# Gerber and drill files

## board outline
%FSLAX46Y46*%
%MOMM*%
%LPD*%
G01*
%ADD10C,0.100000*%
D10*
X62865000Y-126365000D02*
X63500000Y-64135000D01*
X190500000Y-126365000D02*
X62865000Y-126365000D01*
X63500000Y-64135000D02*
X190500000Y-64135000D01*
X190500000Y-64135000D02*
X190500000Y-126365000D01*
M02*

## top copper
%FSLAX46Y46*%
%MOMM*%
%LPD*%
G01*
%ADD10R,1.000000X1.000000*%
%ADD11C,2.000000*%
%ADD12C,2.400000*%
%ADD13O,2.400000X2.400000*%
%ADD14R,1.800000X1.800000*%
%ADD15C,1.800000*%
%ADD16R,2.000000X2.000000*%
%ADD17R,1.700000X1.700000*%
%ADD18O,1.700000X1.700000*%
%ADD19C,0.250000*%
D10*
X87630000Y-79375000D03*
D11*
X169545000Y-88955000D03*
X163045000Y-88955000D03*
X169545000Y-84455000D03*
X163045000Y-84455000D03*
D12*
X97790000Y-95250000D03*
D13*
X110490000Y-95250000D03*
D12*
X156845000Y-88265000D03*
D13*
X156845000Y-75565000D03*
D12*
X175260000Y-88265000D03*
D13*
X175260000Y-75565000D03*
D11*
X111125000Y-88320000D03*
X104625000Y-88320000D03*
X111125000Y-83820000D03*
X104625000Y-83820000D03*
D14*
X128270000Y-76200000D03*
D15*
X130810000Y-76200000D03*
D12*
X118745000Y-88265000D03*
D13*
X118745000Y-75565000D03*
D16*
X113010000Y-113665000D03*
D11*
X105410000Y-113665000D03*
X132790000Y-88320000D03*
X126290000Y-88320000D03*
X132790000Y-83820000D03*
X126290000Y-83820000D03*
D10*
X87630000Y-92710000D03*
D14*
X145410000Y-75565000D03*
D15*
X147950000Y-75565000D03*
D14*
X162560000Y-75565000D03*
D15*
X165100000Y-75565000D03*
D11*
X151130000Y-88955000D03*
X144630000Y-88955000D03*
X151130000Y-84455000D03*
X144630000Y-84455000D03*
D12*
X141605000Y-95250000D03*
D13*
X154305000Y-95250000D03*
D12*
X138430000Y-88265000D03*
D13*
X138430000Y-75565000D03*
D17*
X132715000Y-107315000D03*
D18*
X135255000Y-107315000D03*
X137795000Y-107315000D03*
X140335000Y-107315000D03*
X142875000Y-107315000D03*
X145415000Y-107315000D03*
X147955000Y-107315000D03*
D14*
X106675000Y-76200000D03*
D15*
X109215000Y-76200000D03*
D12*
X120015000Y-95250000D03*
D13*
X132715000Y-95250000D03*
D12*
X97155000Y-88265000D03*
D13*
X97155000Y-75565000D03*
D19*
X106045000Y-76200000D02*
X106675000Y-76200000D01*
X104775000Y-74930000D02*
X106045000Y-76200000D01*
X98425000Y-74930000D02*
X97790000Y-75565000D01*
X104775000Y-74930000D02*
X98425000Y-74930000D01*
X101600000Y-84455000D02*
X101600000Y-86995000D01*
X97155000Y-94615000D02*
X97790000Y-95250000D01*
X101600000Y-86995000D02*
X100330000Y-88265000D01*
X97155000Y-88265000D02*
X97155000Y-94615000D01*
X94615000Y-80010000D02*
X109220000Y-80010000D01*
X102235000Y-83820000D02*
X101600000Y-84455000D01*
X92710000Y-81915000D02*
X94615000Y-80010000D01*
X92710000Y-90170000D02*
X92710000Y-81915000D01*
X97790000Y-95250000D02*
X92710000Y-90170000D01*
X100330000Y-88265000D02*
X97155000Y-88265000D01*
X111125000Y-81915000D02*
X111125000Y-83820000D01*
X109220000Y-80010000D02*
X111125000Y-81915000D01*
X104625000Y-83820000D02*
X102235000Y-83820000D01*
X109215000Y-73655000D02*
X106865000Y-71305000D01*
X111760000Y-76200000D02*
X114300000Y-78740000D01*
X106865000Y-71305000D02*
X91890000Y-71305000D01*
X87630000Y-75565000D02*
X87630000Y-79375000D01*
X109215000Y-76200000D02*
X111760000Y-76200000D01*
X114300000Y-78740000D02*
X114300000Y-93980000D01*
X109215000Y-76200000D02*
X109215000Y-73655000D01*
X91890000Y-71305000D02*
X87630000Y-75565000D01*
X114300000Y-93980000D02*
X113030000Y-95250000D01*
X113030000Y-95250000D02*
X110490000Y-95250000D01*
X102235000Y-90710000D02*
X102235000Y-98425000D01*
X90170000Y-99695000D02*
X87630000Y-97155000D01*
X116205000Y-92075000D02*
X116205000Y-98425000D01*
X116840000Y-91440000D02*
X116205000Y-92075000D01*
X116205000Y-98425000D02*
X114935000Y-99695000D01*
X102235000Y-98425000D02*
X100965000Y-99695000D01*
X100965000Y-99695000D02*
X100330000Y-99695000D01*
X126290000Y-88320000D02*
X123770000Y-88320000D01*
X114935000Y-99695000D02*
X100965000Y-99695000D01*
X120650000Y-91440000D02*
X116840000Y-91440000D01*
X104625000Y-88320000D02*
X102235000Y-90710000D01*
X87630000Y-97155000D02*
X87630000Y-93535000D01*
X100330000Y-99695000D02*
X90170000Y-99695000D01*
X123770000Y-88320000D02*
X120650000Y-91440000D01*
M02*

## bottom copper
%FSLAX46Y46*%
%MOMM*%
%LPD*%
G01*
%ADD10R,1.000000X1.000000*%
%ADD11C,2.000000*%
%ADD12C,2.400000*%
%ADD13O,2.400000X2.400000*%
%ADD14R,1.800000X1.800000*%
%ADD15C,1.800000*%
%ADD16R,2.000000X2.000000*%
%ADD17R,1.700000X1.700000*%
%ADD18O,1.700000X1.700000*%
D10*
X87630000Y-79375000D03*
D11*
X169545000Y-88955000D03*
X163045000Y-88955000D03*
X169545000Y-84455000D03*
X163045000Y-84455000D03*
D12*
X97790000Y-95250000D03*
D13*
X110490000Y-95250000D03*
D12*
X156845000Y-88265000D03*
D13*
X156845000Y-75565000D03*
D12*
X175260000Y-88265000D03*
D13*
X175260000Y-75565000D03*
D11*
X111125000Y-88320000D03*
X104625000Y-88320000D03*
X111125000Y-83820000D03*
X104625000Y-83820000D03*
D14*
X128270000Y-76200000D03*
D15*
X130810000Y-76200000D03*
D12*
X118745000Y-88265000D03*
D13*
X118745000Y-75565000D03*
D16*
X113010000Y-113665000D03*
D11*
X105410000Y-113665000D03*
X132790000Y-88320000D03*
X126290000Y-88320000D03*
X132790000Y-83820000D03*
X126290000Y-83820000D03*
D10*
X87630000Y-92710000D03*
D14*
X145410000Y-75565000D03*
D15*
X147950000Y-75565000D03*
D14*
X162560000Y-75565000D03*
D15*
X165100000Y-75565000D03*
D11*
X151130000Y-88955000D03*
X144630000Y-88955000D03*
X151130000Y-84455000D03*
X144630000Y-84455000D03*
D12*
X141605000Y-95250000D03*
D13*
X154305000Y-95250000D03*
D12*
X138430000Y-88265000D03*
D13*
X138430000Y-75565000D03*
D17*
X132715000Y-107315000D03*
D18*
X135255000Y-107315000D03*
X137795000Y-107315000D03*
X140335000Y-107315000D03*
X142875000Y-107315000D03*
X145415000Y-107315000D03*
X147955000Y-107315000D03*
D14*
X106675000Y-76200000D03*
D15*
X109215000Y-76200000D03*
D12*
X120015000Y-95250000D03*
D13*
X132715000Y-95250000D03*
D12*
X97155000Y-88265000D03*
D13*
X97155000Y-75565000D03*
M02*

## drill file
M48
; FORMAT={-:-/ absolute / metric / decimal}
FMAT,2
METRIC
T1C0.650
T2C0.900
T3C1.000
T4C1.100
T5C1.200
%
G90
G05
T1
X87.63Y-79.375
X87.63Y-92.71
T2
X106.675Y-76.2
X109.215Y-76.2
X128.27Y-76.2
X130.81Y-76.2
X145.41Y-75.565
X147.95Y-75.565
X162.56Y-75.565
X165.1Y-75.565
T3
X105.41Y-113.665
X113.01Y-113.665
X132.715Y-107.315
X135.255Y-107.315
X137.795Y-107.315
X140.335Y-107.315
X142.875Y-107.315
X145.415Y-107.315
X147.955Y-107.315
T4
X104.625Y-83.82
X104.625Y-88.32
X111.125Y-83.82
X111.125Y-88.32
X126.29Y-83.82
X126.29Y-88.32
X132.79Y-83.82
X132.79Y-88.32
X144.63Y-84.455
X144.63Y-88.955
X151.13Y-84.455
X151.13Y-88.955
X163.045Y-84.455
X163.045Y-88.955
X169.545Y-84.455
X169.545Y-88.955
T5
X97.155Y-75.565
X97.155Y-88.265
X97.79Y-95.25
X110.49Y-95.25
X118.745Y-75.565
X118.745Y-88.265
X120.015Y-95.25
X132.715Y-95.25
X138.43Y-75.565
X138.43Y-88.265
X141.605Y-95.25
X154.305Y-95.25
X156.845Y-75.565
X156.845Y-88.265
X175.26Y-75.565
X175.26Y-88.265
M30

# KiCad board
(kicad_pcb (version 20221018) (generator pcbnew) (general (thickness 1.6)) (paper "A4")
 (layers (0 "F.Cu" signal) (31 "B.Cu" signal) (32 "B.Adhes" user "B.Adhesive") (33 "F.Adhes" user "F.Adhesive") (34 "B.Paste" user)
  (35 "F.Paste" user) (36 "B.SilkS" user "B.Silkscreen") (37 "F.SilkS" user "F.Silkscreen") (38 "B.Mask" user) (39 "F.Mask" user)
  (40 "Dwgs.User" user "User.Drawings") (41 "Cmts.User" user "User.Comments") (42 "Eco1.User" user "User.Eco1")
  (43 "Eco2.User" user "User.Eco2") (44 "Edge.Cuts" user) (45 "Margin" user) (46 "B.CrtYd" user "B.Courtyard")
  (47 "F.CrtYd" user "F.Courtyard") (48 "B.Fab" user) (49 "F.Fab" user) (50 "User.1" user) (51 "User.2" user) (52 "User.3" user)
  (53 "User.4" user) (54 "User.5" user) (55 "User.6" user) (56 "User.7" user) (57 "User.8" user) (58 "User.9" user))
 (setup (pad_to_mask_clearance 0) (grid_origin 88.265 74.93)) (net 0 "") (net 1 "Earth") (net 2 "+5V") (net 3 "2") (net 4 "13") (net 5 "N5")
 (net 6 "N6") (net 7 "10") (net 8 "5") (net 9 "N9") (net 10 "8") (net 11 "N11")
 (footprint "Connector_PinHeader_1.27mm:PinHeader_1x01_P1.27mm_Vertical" (layer "F.Cu") (at 87.63 79.375)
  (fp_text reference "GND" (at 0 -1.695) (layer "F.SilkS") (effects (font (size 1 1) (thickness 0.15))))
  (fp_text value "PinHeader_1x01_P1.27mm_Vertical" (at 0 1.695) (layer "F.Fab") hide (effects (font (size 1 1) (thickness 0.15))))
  (pad "1" thru_hole rect (at 0 0) (size 1 1) (drill 0.65) (layers "*.Cu" "*.Mask") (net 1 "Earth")))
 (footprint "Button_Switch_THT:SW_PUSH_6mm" (layer "F.Cu") (at 169.545 88.955 180)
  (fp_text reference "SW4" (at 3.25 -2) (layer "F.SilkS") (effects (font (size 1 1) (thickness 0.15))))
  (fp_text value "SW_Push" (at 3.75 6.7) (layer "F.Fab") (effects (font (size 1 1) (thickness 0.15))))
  (pad "1" thru_hole circle (at 0 0 270) (size 2 2) (drill 1.1) (layers "*.Cu" "*.Mask") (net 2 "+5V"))
  (pad "1" thru_hole circle (at 6.5 0 270) (size 2 2) (drill 1.1) (layers "*.Cu" "*.Mask") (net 2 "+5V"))
  (pad "2" thru_hole circle (at 0 4.5 270) (size 2 2) (drill 1.1) (layers "*.Cu" "*.Mask") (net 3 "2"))
  (pad "2" thru_hole circle (at 6.5 4.5 270) (size 2 2) (drill 1.1) (layers "*.Cu" "*.Mask") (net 3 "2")))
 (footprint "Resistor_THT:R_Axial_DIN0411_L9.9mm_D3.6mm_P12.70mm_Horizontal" (layer "F.Cu") (at 97.79 95.25)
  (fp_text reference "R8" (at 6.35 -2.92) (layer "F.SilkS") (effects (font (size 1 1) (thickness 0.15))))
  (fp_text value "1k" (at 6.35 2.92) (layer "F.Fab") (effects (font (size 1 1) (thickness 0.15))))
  (pad "1" thru_hole circle (at 0 0) (size 2.4 2.4) (drill 1.2) (layers "*.Cu" "*.Mask") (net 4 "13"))
  (pad "2" thru_hole oval (at 12.7 0) (size 2.4 2.4) (drill 1.2) (layers "*.Cu" "*.Mask") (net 1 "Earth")))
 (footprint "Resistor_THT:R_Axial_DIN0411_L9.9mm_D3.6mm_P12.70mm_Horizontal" (layer "F.Cu") (at 156.845 88.265 90)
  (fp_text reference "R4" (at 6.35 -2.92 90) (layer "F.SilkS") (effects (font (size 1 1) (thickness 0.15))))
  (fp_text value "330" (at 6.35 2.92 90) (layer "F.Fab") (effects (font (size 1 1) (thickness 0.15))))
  (pad "1" thru_hole circle (at 0 0 90) (size 2.4 2.4) (drill 1.2) (layers "*.Cu" "*.Mask") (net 3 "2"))
  (pad "2" thru_hole oval (at 12.7 0 90) (size 2.4 2.4) (drill 1.2) (layers "*.Cu" "*.Mask") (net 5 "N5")))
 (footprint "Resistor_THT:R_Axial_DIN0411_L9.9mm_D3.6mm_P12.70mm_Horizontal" (layer "F.Cu") (at 175.26 88.265 90)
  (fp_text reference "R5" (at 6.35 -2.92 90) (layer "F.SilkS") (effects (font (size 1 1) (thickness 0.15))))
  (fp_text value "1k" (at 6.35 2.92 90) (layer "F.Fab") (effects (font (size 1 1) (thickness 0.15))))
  (pad "1" thru_hole circle (at 0 0 90) (size 2.4 2.4) (drill 1.2) (layers "*.Cu" "*.Mask") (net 3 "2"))
  (pad "2" thru_hole oval (at 12.7 0 90) (size 2.4 2.4) (drill 1.2) (layers "*.Cu" "*.Mask") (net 1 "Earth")))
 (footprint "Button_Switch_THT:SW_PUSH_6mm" (layer "F.Cu") (at 111.125 88.32 180)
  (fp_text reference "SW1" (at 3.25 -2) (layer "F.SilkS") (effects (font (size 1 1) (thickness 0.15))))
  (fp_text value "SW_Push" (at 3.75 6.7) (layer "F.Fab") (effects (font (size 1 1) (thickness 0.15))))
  (pad "1" thru_hole circle (at 0 0 270) (size 2 2) (drill 1.1) (layers "*.Cu" "*.Mask") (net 2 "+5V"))
  (pad "1" thru_hole circle (at 6.5 0 270) (size 2 2) (drill 1.1) (layers "*.Cu" "*.Mask") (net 2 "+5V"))
  (pad "2" thru_hole circle (at 0 4.5 270) (size 2 2) (drill 1.1) (layers "*.Cu" "*.Mask") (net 4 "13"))
  (pad "2" thru_hole circle (at 6.5 4.5 270) (size 2 2) (drill 1.1) (layers "*.Cu" "*.Mask") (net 4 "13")))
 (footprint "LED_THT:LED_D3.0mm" (layer "F.Cu") (at 128.27 76.2)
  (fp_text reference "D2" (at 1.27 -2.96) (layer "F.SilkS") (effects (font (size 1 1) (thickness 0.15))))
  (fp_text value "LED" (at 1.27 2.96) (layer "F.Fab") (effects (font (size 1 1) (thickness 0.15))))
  (pad "1" thru_hole rect (at 0 0) (size 1.8 1.8) (drill 0.9) (layers "*.Cu" "*.Mask") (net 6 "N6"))
  (pad "2" thru_hole circle (at 2.54 0) (size 1.8 1.8) (drill 0.9) (layers "*.Cu" "*.Mask") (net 1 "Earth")))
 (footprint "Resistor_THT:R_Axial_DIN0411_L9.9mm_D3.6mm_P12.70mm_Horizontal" (layer "F.Cu") (at 118.745 88.265 90)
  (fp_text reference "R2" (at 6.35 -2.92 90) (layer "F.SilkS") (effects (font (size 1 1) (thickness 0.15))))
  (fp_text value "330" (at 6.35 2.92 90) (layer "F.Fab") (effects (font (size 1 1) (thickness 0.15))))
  (pad "1" thru_hole circle (at 0 0 90) (size 2.4 2.4) (drill 1.2) (layers "*.Cu" "*.Mask") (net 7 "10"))
  (pad "2" thru_hole oval (at 12.7 0 90) (size 2.4 2.4) (drill 1.2) (layers "*.Cu" "*.Mask") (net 6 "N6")))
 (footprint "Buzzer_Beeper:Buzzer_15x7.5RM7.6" (layer "F.Cu") (at 113.01 113.665 180)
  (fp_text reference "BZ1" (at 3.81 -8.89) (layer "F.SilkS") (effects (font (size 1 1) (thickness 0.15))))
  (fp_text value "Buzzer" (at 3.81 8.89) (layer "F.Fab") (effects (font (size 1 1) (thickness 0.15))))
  (pad "1" thru_hole rect (at 0 0 180) (size 2 2) (drill 1) (layers "*.Cu" "*.Mask") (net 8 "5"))
  (pad "2" thru_hole circle (at 7.6 0 180) (size 2 2) (drill 1) (layers "*.Cu" "*.Mask") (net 1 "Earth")))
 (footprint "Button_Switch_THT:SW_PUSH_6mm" (layer "F.Cu") (at 132.79 88.32 180)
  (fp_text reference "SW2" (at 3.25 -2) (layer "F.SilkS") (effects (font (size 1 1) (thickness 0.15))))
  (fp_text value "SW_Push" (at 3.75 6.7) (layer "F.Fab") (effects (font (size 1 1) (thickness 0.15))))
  (pad "1" thru_hole circle (at 0 0 270) (size 2 2) (drill 1.1) (layers "*.Cu" "*.Mask") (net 2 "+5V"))
  (pad "1" thru_hole circle (at 6.5 0 270) (size 2 2) (drill 1.1) (layers "*.Cu" "*.Mask") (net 2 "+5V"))
  (pad "2" thru_hole circle (at 0 4.5 270) (size 2 2) (drill 1.1) (layers "*.Cu" "*.Mask") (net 7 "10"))
  (pad "2" thru_hole circle (at 6.5 4.5 270) (size 2 2) (drill 1.1) (layers "*.Cu" "*.Mask") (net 7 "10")))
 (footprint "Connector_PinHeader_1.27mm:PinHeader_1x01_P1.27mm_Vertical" (layer "F.Cu") (at 87.63 92.71)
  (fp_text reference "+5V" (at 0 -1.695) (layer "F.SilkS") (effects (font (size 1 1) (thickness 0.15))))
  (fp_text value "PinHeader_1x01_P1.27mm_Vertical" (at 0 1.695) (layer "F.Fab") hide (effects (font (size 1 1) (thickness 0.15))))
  (pad "1" thru_hole rect (at 0 0) (size 1 1) (drill 0.65) (layers "*.Cu" "*.Mask")))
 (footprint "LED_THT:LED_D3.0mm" (layer "F.Cu") (at 145.41 75.565)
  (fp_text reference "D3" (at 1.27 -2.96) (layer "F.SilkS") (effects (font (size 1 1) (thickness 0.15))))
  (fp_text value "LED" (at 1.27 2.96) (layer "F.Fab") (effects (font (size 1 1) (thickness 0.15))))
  (pad "1" thru_hole rect (at 0 0) (size 1.8 1.8) (drill 0.9) (layers "*.Cu" "*.Mask") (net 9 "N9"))
  (pad "2" thru_hole circle (at 2.54 0) (size 1.8 1.8) (drill 0.9) (layers "*.Cu" "*.Mask") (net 1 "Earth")))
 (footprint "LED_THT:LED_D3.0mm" (layer "F.Cu") (at 162.56 75.565)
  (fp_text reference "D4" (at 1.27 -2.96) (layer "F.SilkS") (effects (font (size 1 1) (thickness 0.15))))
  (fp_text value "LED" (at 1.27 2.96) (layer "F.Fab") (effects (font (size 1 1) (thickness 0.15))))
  (pad "1" thru_hole rect (at 0 0) (size 1.8 1.8) (drill 0.9) (layers "*.Cu" "*.Mask") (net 5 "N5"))
  (pad "2" thru_hole circle (at 2.54 0) (size 1.8 1.8) (drill 0.9) (layers "*.Cu" "*.Mask") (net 1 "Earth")))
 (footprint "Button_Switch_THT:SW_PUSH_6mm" (layer "F.Cu") (at 151.13 88.955 180)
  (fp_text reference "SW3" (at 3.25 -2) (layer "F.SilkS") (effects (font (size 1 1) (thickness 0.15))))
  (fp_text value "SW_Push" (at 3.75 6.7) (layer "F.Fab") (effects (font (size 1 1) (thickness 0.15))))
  (pad "1" thru_hole circle (at 0 0 270) (size 2 2) (drill 1.1) (layers "*.Cu" "*.Mask") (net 2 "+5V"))
  (pad "1" thru_hole circle (at 6.5 0 270) (size 2 2) (drill 1.1) (layers "*.Cu" "*.Mask") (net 2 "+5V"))
  (pad "2" thru_hole circle (at 0 4.5 270) (size 2 2) (drill 1.1) (layers "*.Cu" "*.Mask") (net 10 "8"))
  (pad "2" thru_hole circle (at 6.5 4.5 270) (size 2 2) (drill 1.1) (layers "*.Cu" "*.Mask") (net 10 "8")))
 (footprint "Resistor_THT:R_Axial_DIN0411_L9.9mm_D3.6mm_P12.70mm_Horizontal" (layer "F.Cu") (at 141.605 95.25)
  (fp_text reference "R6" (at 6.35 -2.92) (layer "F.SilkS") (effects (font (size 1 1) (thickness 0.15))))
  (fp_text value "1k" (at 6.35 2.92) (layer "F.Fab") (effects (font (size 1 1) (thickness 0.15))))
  (pad "1" thru_hole circle (at 0 0) (size 2.4 2.4) (drill 1.2) (layers "*.Cu" "*.Mask") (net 10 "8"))
  (pad "2" thru_hole oval (at 12.7 0) (size 2.4 2.4) (drill 1.2) (layers "*.Cu" "*.Mask") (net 1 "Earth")))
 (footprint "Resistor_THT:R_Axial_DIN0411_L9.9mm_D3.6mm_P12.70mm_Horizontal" (layer "F.Cu") (at 138.43 88.265 90)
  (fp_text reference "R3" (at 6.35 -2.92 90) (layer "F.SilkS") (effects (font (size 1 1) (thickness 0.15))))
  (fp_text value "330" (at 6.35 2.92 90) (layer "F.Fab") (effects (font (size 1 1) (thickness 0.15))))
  (pad "1" thru_hole circle (at 0 0 90) (size 2.4 2.4) (drill 1.2) (layers "*.Cu" "*.Mask") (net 10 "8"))
  (pad "2" thru_hole oval (at 12.7 0 90) (size 2.4 2.4) (drill 1.2) (layers "*.Cu" "*.Mask") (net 9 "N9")))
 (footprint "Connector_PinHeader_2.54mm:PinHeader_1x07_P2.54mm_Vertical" (layer "F.Cu") (at 132.715 107.315 90)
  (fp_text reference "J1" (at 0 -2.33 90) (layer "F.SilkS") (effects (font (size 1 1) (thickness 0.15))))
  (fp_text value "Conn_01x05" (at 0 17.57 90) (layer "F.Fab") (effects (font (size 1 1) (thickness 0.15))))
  (pad "1" thru_hole rect (at 0 0 90) (size 1.7 1.7) (drill 1) (layers "*.Cu" "*.Mask") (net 4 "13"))
  (pad "2" thru_hole oval (at 0 2.54 90) (size 1.7 1.7) (drill 1) (layers "*.Cu" "*.Mask") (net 7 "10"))
  (pad "3" thru_hole oval (at 0 5.08 90) (size 1.7 1.7) (drill 1) (layers "*.Cu" "*.Mask") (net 10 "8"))
  (pad "4" thru_hole oval (at 0 7.62 90) (size 1.7 1.7) (drill 1) (layers "*.Cu" "*.Mask") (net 8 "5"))
  (pad "5" thru_hole oval (at 0 10.16 90) (size 1.7 1.7) (drill 1) (layers "*.Cu" "*.Mask") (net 3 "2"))
  (pad "6" thru_hole oval (at 0 12.7 90) (size 1.7 1.7) (drill 1) (layers "*.Cu" "*.Mask"))
  (pad "7" thru_hole oval (at 0 15.24 90) (size 1.7 1.7) (drill 1) (layers "*.Cu" "*.Mask")))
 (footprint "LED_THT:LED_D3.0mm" (layer "F.Cu") (at 106.675 76.2)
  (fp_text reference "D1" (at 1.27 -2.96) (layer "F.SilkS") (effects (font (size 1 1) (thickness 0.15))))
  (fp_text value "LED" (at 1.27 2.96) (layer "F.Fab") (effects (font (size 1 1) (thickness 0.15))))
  (pad "1" thru_hole rect (at 0 0) (size 1.8 1.8) (drill 0.9) (layers "*.Cu" "*.Mask") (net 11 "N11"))
  (pad "2" thru_hole circle (at 2.54 0) (size 1.8 1.8) (drill 0.9) (layers "*.Cu" "*.Mask") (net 1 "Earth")))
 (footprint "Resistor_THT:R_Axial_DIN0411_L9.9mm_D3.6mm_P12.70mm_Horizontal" (layer "F.Cu") (at 120.015 95.25)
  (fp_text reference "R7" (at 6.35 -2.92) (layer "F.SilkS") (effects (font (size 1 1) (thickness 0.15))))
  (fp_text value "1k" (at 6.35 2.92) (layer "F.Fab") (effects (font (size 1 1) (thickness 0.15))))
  (pad "1" thru_hole circle (at 0 0) (size 2.4 2.4) (drill 1.2) (layers "*.Cu" "*.Mask") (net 7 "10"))
  (pad "2" thru_hole oval (at 12.7 0) (size 2.4 2.4) (drill 1.2) (layers "*.Cu" "*.Mask") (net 1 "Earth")))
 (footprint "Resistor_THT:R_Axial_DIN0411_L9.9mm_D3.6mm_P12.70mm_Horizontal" (layer "F.Cu") (at 97.155 88.265 90)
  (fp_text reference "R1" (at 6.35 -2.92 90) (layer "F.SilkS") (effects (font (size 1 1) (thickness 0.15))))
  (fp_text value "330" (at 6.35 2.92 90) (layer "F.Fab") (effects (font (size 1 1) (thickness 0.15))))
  (pad "1" thru_hole circle (at 0 0 90) (size 2.4 2.4) (drill 1.2) (layers "*.Cu" "*.Mask") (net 4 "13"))
  (pad "2" thru_hole oval (at 12.7 0 90) (size 2.4 2.4) (drill 1.2) (layers "*.Cu" "*.Mask") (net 11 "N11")))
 (gr_line (start 62.865 126.365) (end 63.5 64.135) (stroke (width 0.1) (type default)) (layer "Edge.Cuts"))
 (gr_line (start 190.5 126.365) (end 62.865 126.365) (stroke (width 0.1) (type default)) (layer "Edge.Cuts"))
 (gr_line (start 63.5 64.135) (end 190.5 64.135) (stroke (width 0.1) (type default)) (layer "Edge.Cuts"))
 (gr_line (start 190.5 64.135) (end 190.5 126.365) (stroke (width 0.1) (type default)) (layer "Edge.Cuts"))
 (segment (start 106.045 76.2) (end 106.675 76.2) (width 0.25) (layer "F.Cu") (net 11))
 (segment (start 104.775 74.93) (end 106.045 76.2) (width 0.25) (layer "F.Cu") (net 11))
 (segment (start 98.425 74.93) (end 97.79 75.565) (width 0.25) (layer "F.Cu") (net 11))
 (segment (start 104.775 74.93) (end 98.425 74.93) (width 0.25) (layer "F.Cu") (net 11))
 (segment (start 101.6 84.455) (end 101.6 86.995) (width 0.25) (layer "F.Cu") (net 4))
 (segment (start 97.155 94.615) (end 97.79 95.25) (width 0.25) (layer "F.Cu") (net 4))
 (segment (start 101.6 86.995) (end 100.33 88.265) (width 0.25) (layer "F.Cu") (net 4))
 (segment (start 97.155 88.265) (end 97.155 94.615) (width 0.25) (layer "F.Cu") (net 4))
 (segment (start 94.615 80.01) (end 109.22 80.01) (width 0.25) (layer "F.Cu") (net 4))
 (segment (start 102.235 83.82) (end 101.6 84.455) (width 0.25) (layer "F.Cu") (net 4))
 (segment (start 92.71 81.915) (end 94.615 80.01) (width 0.25) (layer "F.Cu") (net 4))
 (segment (start 92.71 90.17) (end 92.71 81.915) (width 0.25) (layer "F.Cu") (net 4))
 (segment (start 97.79 95.25) (end 92.71 90.17) (width 0.25) (layer "F.Cu") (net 4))
 (segment (start 100.33 88.265) (end 97.155 88.265) (width 0.25) (layer "F.Cu") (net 4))
 (segment (start 111.125 81.915) (end 111.125 83.82) (width 0.25) (layer "F.Cu") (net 4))
 (segment (start 109.22 80.01) (end 111.125 81.915) (width 0.25) (layer "F.Cu") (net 4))
 (segment (start 104.625 83.82) (end 102.235 83.82) (width 0.25) (layer "F.Cu") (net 4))
 (segment (start 109.215 73.655) (end 106.865 71.305) (width 0.25) (layer "F.Cu") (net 1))
 (segment (start 111.76 76.2) (end 114.3 78.74) (width 0.25) (layer "F.Cu") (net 1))
 (segment (start 106.865 71.305) (end 91.89 71.305) (width 0.25) (layer "F.Cu") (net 1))
 (segment (start 87.63 75.565) (end 87.63 79.375) (width 0.25) (layer "F.Cu") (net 1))
 (segment (start 109.215 76.2) (end 111.76 76.2) (width 0.25) (layer "F.Cu") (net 1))
 (segment (start 114.3 78.74) (end 114.3 93.98) (width 0.25) (layer "F.Cu") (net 1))
 (segment (start 109.215 76.2) (end 109.215 73.655) (width 0.25) (layer "F.Cu") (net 1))
 (segment (start 91.89 71.305) (end 87.63 75.565) (width 0.25) (layer "F.Cu") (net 1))
 (segment (start 114.3 93.98) (end 113.03 95.25) (width 0.25) (layer "F.Cu") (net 1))
 (segment (start 113.03 95.25) (end 110.49 95.25) (width 0.25) (layer "F.Cu") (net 1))
 (segment (start 102.235 90.71) (end 102.235 98.425) (width 0.25) (layer "F.Cu") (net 2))
 (segment (start 90.17 99.695) (end 87.63 97.155) (width 0.25) (layer "F.Cu") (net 2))
 (segment (start 116.205 92.075) (end 116.205 98.425) (width 0.25) (layer "F.Cu") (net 2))
 (segment (start 116.84 91.44) (end 116.205 92.075) (width 0.25) (layer "F.Cu") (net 2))
 (segment (start 116.205 98.425) (end 114.935 99.695) (width 0.25) (layer "F.Cu") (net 2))
 (segment (start 102.235 98.425) (end 100.965 99.695) (width 0.25) (layer "F.Cu") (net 2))
 (segment (start 100.965 99.695) (end 100.33 99.695) (width 0.25) (layer "F.Cu") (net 2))
 (segment (start 126.29 88.32) (end 123.77 88.32) (width 0.25) (layer "F.Cu") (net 2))
 (segment (start 114.935 99.695) (end 100.965 99.695) (width 0.25) (layer "F.Cu") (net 2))
 (segment (start 120.65 91.44) (end 116.84 91.44) (width 0.25) (layer "F.Cu") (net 2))
 (segment (start 104.625 88.32) (end 102.235 90.71) (width 0.25) (layer "F.Cu") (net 2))
 (segment (start 87.63 97.155) (end 87.63 93.535) (width 0.25) (layer "F.Cu") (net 2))
 (segment (start 100.33 99.695) (end 90.17 99.695) (width 0.25) (layer "F.Cu") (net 2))
 (segment (start 123.77 88.32) (end 120.65 91.44) (width 0.25) (layer "F.Cu") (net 2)))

